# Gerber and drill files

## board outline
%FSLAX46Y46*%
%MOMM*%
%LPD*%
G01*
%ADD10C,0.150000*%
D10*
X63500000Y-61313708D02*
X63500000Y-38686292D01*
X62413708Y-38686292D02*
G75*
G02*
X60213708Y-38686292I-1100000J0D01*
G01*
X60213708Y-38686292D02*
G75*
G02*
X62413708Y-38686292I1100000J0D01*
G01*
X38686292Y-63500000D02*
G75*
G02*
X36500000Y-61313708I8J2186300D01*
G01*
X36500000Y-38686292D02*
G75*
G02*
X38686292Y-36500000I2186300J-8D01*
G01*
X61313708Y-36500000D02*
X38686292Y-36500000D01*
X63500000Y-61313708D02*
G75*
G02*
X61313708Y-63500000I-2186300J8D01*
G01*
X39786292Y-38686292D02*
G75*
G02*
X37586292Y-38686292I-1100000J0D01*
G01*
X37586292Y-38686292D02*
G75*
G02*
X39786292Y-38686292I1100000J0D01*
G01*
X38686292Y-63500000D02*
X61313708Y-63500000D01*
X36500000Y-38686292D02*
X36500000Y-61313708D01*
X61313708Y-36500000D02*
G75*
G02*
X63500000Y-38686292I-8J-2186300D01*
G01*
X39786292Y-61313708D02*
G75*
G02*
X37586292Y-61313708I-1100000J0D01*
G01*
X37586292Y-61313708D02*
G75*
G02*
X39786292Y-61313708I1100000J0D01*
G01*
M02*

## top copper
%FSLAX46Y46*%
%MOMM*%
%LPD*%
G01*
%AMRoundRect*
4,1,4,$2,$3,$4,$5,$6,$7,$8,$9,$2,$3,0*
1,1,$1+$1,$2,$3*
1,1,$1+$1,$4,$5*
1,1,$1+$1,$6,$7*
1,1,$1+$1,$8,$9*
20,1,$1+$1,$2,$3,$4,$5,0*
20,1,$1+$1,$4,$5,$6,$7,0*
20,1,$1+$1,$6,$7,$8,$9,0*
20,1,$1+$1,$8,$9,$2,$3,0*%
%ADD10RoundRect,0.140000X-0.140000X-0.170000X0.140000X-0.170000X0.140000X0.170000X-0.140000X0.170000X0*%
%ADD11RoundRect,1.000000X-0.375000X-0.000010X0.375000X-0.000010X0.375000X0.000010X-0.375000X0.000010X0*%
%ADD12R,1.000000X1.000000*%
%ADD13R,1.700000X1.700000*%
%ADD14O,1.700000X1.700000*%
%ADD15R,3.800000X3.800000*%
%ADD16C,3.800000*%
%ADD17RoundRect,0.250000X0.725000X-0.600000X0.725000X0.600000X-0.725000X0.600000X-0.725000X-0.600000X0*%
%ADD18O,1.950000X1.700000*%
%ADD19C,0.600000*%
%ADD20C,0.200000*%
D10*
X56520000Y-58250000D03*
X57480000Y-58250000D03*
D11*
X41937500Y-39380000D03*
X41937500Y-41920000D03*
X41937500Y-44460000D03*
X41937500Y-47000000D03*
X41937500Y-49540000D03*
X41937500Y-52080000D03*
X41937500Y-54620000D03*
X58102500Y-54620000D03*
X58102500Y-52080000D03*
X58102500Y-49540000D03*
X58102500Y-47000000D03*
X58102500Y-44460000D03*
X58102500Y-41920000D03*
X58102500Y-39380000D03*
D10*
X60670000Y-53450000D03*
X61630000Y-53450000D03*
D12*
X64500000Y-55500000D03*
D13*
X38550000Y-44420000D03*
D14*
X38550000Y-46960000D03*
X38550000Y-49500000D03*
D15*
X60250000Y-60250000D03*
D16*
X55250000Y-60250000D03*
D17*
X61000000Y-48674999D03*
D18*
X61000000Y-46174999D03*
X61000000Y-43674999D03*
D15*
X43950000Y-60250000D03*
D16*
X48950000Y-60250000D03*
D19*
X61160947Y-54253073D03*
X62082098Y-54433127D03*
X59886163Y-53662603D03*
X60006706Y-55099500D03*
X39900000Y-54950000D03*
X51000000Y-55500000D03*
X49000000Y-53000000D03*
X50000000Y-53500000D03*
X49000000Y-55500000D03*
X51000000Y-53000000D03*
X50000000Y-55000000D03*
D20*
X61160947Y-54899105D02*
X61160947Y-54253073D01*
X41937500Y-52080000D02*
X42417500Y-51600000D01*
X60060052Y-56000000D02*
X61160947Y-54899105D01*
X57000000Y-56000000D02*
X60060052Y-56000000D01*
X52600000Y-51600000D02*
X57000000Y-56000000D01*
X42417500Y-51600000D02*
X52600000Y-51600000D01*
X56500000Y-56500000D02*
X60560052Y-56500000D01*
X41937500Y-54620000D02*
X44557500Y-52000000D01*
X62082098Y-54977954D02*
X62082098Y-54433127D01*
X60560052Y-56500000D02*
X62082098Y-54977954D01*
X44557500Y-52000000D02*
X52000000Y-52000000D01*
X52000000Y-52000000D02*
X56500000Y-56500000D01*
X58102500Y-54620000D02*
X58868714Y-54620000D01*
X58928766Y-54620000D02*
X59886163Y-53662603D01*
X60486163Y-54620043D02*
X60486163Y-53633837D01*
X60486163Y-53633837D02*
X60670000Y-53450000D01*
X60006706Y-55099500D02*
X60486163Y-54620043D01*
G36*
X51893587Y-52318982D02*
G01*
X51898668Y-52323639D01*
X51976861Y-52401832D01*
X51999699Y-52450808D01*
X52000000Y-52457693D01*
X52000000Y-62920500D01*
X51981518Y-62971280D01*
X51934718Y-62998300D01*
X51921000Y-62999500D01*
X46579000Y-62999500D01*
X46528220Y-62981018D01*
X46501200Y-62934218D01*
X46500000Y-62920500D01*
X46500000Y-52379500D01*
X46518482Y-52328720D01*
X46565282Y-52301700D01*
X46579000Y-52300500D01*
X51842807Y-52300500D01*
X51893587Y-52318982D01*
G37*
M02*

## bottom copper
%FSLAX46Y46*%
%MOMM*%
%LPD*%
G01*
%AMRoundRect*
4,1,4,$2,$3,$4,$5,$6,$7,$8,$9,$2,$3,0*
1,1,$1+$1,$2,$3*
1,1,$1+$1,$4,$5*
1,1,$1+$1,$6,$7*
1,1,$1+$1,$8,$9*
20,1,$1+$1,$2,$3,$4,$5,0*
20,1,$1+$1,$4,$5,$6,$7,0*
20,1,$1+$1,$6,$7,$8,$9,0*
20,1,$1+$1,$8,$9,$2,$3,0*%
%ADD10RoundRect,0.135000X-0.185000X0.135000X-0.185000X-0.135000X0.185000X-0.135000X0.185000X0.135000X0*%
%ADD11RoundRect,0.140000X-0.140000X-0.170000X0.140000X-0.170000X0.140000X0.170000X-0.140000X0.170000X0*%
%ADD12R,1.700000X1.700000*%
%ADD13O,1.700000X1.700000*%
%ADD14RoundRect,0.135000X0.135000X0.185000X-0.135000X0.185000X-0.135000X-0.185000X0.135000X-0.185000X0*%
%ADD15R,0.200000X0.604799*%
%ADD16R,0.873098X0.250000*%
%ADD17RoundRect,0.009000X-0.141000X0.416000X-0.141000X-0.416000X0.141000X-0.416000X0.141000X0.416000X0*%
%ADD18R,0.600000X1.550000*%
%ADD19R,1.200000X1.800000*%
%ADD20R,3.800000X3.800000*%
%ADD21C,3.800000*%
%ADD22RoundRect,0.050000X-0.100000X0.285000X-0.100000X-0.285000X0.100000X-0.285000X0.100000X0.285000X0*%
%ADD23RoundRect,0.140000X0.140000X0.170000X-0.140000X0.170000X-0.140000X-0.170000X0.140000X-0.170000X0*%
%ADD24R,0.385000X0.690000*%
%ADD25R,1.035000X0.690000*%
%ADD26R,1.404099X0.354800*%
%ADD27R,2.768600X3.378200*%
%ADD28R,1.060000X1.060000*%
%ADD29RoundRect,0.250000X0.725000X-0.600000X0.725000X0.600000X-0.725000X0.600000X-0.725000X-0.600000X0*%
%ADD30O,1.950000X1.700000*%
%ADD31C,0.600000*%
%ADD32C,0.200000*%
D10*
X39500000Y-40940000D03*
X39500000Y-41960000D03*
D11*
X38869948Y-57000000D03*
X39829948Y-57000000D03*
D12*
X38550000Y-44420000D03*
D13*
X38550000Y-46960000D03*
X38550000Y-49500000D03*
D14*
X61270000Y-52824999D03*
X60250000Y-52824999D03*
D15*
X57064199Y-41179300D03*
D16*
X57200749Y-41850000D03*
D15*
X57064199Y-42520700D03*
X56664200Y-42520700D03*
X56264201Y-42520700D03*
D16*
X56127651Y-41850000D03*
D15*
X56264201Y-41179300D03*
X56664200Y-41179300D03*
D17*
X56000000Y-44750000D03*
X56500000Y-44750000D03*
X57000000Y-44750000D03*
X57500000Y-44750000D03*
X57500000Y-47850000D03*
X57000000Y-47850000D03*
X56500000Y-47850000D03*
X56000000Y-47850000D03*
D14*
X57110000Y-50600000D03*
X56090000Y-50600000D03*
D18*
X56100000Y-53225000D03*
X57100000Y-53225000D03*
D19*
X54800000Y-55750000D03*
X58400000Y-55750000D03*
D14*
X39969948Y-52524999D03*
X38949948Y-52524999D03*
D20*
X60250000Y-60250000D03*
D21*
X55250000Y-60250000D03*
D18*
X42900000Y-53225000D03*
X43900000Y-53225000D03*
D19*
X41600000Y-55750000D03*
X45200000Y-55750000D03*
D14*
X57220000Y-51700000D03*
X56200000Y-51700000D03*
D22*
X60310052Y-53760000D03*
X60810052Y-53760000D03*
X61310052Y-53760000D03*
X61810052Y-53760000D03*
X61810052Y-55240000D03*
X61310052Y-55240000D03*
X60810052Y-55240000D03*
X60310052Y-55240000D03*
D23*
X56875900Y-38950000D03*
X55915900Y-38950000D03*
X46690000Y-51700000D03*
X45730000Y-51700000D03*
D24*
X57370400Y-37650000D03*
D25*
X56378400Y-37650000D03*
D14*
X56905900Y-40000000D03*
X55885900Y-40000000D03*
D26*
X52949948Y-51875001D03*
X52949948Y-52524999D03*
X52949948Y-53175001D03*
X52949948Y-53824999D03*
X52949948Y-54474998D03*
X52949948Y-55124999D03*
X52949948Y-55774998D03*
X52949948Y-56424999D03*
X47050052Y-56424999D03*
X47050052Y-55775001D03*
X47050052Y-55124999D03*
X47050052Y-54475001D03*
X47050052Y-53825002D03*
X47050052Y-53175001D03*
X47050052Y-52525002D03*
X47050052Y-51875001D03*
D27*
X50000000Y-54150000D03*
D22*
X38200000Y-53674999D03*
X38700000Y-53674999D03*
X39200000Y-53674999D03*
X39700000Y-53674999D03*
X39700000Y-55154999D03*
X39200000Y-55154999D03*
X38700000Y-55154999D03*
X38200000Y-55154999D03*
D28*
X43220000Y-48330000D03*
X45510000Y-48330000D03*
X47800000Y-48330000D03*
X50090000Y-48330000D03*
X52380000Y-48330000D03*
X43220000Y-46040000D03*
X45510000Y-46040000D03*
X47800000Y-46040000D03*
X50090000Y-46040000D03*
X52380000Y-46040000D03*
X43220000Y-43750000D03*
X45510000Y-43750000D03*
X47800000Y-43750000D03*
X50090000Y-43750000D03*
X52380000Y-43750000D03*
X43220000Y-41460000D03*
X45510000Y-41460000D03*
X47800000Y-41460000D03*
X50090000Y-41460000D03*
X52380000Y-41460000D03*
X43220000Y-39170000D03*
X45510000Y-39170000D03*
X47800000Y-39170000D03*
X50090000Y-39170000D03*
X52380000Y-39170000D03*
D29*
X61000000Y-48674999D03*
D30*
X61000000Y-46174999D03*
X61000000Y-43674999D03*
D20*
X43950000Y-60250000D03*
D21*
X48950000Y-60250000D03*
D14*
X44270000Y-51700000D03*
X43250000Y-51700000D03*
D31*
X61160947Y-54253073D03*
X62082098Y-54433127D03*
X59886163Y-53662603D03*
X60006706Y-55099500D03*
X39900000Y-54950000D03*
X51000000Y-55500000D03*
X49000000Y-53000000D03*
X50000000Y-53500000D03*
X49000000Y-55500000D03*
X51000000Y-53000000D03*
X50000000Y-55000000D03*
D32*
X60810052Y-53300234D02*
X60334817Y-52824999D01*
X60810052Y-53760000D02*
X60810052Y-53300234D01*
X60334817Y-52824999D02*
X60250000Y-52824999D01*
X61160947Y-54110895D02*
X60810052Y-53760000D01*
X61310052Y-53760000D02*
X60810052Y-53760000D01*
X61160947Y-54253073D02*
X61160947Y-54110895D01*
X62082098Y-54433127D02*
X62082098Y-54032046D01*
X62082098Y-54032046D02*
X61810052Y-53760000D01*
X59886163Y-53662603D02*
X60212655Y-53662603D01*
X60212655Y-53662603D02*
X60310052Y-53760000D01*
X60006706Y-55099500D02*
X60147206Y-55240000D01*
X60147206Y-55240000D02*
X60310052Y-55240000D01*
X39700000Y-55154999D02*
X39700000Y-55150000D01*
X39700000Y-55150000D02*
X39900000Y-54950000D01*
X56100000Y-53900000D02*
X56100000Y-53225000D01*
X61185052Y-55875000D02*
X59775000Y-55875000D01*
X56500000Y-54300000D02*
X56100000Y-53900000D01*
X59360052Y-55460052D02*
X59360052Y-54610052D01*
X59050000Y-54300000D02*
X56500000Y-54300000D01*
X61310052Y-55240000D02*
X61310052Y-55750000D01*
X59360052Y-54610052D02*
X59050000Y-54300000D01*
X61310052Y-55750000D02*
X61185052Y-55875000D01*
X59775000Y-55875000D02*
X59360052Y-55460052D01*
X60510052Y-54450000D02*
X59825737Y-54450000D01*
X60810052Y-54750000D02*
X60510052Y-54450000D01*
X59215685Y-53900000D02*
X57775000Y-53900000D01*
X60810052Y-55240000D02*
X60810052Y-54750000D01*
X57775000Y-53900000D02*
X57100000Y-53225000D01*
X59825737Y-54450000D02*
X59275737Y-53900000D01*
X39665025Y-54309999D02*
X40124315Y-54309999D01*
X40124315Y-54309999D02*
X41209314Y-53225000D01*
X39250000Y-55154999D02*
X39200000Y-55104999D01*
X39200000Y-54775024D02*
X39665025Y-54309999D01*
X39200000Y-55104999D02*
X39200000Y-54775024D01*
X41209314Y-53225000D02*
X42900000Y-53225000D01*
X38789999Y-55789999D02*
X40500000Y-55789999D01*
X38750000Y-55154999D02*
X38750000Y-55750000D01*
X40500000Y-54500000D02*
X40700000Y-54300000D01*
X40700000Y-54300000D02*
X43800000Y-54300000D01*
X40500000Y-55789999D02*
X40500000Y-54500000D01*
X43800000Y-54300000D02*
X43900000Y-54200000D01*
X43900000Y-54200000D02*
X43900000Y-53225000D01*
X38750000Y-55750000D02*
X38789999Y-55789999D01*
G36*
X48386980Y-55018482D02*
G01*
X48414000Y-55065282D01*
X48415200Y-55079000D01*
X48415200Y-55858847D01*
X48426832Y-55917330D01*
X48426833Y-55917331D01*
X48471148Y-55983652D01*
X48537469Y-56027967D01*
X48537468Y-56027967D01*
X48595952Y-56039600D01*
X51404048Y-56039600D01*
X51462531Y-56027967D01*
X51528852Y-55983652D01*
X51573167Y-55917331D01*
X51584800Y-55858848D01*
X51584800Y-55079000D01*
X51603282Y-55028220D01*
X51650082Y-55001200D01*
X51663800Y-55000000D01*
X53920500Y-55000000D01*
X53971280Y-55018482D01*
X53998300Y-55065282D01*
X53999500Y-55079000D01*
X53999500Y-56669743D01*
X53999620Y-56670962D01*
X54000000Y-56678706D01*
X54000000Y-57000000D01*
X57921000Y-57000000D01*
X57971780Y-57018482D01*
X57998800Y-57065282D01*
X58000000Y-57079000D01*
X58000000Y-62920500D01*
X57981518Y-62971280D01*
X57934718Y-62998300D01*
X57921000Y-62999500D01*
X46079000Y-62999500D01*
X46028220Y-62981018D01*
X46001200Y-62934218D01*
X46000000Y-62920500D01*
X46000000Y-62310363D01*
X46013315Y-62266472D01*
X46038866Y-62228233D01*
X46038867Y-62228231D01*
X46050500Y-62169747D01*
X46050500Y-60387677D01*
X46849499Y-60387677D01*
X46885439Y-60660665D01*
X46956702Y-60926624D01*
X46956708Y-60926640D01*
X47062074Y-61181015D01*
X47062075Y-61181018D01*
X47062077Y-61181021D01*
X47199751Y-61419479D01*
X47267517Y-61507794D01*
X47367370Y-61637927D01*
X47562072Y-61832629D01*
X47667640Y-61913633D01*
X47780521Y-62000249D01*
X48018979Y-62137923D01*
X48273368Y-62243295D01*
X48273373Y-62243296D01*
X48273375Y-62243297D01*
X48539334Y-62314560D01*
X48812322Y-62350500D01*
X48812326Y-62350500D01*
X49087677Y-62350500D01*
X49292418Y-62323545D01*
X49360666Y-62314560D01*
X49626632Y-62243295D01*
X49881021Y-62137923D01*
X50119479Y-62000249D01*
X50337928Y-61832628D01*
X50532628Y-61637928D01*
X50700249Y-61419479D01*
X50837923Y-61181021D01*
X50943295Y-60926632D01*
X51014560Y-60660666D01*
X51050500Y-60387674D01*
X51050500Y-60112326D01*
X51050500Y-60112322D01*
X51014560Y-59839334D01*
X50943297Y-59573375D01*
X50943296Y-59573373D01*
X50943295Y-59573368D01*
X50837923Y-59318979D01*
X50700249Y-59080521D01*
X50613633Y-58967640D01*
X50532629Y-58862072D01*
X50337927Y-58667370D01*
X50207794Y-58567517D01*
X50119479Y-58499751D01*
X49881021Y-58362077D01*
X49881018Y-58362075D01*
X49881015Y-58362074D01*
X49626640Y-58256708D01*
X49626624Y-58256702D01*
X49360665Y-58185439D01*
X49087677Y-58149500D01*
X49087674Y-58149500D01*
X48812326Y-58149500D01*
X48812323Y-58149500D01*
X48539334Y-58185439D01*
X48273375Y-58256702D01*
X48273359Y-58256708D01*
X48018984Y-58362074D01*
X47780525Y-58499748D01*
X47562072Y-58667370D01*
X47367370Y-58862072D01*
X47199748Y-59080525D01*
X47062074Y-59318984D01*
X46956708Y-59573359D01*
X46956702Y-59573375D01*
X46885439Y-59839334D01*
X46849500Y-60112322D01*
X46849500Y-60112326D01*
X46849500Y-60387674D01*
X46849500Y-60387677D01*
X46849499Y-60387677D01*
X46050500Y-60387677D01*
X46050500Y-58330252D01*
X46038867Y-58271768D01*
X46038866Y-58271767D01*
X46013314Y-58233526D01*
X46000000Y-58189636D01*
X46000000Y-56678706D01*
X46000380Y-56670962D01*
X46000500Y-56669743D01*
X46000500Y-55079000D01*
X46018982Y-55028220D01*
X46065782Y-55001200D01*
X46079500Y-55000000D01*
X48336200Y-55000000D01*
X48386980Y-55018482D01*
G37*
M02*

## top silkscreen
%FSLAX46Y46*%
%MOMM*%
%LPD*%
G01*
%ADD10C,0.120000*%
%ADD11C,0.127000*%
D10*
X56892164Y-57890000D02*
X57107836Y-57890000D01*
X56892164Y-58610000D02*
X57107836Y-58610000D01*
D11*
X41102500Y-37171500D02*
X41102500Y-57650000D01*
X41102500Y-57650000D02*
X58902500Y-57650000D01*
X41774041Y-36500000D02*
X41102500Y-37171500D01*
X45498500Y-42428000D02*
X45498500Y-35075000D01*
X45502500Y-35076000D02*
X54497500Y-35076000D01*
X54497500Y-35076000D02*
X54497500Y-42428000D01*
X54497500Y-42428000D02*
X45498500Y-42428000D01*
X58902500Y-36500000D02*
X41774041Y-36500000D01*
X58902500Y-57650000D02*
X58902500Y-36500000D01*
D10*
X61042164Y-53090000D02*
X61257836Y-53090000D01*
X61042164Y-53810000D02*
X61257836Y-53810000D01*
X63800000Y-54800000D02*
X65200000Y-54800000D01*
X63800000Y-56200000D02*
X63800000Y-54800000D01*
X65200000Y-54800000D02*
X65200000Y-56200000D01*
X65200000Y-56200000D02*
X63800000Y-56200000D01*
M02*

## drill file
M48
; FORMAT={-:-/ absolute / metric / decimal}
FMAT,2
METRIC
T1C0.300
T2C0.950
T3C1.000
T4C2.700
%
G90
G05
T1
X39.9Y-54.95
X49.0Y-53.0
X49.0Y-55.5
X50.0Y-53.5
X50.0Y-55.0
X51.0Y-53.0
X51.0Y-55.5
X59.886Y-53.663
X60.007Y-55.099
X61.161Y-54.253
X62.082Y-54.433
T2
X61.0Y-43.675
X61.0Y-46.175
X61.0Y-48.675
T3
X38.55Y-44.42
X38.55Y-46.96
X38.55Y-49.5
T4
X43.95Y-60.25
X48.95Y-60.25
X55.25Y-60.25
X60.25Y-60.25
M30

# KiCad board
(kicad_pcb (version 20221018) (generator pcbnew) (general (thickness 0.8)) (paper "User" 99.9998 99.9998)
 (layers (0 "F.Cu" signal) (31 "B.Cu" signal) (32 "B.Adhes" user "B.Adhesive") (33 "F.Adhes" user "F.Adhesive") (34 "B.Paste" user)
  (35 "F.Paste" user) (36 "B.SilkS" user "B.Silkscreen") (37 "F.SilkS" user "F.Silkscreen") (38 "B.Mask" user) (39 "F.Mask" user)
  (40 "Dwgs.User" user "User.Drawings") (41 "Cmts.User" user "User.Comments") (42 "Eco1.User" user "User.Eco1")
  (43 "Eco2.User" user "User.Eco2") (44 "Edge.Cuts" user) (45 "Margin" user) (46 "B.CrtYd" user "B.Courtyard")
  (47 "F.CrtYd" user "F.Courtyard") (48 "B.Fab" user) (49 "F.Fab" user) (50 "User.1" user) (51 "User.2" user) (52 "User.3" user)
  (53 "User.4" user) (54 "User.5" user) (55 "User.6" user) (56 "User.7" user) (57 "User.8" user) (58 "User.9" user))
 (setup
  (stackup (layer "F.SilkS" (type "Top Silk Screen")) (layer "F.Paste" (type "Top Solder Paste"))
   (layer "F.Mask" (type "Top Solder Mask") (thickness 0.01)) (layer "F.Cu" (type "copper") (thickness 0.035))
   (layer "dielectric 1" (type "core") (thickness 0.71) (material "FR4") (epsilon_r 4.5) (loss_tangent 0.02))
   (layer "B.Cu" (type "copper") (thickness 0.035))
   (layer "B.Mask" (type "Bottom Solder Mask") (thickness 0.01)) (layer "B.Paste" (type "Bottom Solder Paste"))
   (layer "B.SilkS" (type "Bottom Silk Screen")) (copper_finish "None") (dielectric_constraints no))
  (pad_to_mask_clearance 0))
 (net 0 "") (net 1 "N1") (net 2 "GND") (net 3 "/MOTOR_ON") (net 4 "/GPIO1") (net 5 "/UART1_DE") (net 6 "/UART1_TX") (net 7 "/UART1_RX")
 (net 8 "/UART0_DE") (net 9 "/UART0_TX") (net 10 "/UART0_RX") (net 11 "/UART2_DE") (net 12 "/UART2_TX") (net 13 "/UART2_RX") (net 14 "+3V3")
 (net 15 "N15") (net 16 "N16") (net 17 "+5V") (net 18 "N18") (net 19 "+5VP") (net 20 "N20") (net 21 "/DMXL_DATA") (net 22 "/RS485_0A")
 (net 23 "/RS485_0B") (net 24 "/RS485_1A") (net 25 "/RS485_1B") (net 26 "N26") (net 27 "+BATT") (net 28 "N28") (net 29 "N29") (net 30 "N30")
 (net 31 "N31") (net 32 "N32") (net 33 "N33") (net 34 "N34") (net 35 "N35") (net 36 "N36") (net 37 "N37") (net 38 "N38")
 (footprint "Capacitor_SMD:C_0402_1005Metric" (layer "F.Cu") (at 57 58.25)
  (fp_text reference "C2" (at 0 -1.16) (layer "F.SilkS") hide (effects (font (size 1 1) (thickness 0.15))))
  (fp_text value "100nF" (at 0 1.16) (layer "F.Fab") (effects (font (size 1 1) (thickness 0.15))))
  (fp_line (start -0.107836 -0.36) (end 0.107836 -0.36) (stroke (width 0.12) (type solid)) (layer "F.SilkS"))
  (fp_line (start -0.107836 0.36) (end 0.107836 0.36) (stroke (width 0.12) (type solid)) (layer "F.SilkS"))
  (pad "1" smd roundrect (at -0.48 0) (size 0.56 0.62) (layers "F.Cu" "F.Paste" "F.Mask") (roundrect_rratio 0.25) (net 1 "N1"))
  (pad "2" smd roundrect (at 0.48 0) (size 0.56 0.62) (layers "F.Cu" "F.Paste" "F.Mask") (roundrect_rratio 0.25) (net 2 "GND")))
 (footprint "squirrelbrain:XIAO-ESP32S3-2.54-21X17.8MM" (layer "F.Cu") (at 50 36.5)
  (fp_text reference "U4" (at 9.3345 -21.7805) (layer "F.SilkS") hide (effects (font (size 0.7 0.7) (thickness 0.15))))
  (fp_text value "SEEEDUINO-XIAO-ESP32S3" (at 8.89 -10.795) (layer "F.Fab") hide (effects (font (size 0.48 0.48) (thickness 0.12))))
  (fp_line (start -8.8975 0.6715) (end -8.8975 21.15) (stroke (width 0.127) (type solid)) (layer "F.SilkS"))
  (fp_line (start -8.8975 21.15) (end 8.9025 21.15) (stroke (width 0.127) (type solid)) (layer "F.SilkS"))
  (fp_line (start -8.225959 0) (end -8.8975 0.6715) (stroke (width 0.127) (type solid)) (layer "F.SilkS"))
  (fp_line (start -4.5015 5.928) (end -4.5015 -1.425) (stroke (width 0.127) (type solid)) (layer "F.SilkS"))
  (fp_line (start -4.4975 -1.424) (end 4.4975 -1.424) (stroke (width 0.127) (type solid)) (layer "F.SilkS"))
  (fp_line (start 4.4975 -1.424) (end 4.4975 5.928) (stroke (width 0.127) (type solid)) (layer "F.SilkS"))
  (fp_line (start 4.4975 5.928) (end -4.5015 5.928) (stroke (width 0.127) (type solid)) (layer "F.SilkS"))
  (fp_line (start 8.9025 0) (end -8.225959 0) (stroke (width 0.127) (type solid)) (layer "F.SilkS"))
  (fp_line (start 8.9025 21.15) (end 8.9025 0) (stroke (width 0.127) (type solid)) (layer "F.SilkS"))
  (pad "1" smd roundrect (at -8.0625 2.88) (size 2.75 2) (layers "F.Cu" "F.Paste" "F.Mask") (roundrect_rratio 0.5) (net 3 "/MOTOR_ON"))
  (pad "2" smd roundrect (at -8.0625 5.42) (size 2.75 2) (layers "F.Cu" "F.Paste" "F.Mask") (roundrect_rratio 0.5) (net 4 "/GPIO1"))
  (pad "3" smd roundrect (at -8.0625 7.96) (size 2.75 2) (layers "F.Cu" "F.Paste" "F.Mask") (roundrect_rratio 0.5) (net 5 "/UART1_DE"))
  (pad "4" smd roundrect (at -8.0625 10.5) (size 2.75 2) (layers "F.Cu" "F.Paste" "F.Mask") (roundrect_rratio 0.5) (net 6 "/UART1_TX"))
  (pad "5" smd roundrect (at -8.0625 13.04) (size 2.75 2) (layers "F.Cu" "F.Paste" "F.Mask") (roundrect_rratio 0.5) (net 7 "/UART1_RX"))
  (pad "6" smd roundrect (at -8.0625 15.58) (size 2.75 2) (layers "F.Cu" "F.Paste" "F.Mask") (roundrect_rratio 0.5) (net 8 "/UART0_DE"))
  (pad "7" smd roundrect (at -8.0625 18.12) (size 2.75 2) (layers "F.Cu" "F.Paste" "F.Mask") (roundrect_rratio 0.5) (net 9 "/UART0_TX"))
  (pad "8" smd roundrect (at 8.1025 18.12) (size 2.75 2) (layers "F.Cu" "F.Paste" "F.Mask") (roundrect_rratio 0.5) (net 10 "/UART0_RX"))
  (pad "9" smd roundrect (at 8.1025 15.58) (size 2.75 2) (layers "F.Cu" "F.Paste" "F.Mask") (roundrect_rratio 0.5) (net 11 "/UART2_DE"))
  (pad "10" smd roundrect (at 8.1025 13.04) (size 2.75 2) (layers "F.Cu" "F.Paste" "F.Mask") (roundrect_rratio 0.5) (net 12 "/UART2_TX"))
  (pad "11" smd roundrect (at 8.1025 10.5) (size 2.75 2) (layers "F.Cu" "F.Paste" "F.Mask") (roundrect_rratio 0.5) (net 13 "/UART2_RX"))
  (pad "12" smd roundrect (at 8.1025 7.96) (size 2.75 2) (layers "F.Cu" "F.Paste" "F.Mask") (roundrect_rratio 0.5) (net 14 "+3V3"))
  (pad "13" smd roundrect (at 8.1025 5.42) (size 2.75 2) (layers "F.Cu" "F.Paste" "F.Mask") (roundrect_rratio 0.5) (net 2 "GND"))
  (pad "14" smd roundrect (at 8.1025 2.88) (size 2.75 2) (layers "F.Cu" "F.Paste" "F.Mask") (roundrect_rratio 0.5) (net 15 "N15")))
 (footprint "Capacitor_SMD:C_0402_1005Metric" (layer "F.Cu") (at 61.15 53.45)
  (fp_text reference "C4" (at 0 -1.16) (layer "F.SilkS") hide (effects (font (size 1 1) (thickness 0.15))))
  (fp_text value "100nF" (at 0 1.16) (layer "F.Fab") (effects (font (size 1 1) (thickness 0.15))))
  (fp_line (start -0.107836 -0.36) (end 0.107836 -0.36) (stroke (width 0.12) (type solid)) (layer "F.SilkS"))
  (fp_line (start -0.107836 0.36) (end 0.107836 0.36) (stroke (width 0.12) (type solid)) (layer "F.SilkS"))
  (pad "1" smd roundrect (at -0.48 0) (size 0.56 0.62) (layers "F.Cu" "F.Paste" "F.Mask") (roundrect_rratio 0.25) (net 14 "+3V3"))
  (pad "2" smd roundrect (at 0.48 0) (size 0.56 0.62) (layers "F.Cu" "F.Paste" "F.Mask") (roundrect_rratio 0.25) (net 2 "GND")))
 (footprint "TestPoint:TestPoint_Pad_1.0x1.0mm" (layer "F.Cu") (at 64.5 55.5)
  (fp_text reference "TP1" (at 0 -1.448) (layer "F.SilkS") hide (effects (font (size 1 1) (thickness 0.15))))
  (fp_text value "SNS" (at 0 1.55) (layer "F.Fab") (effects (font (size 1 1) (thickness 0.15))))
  (fp_line (start -0.7 -0.7) (end 0.7 -0.7) (stroke (width 0.12) (type solid)) (layer "F.SilkS"))
  (fp_line (start -0.7 0.7) (end -0.7 -0.7) (stroke (width 0.12) (type solid)) (layer "F.SilkS"))
  (fp_line (start 0.7 -0.7) (end 0.7 0.7) (stroke (width 0.12) (type solid)) (layer "F.SilkS"))
  (fp_line (start 0.7 0.7) (end -0.7 0.7) (stroke (width 0.12) (type solid)) (layer "F.SilkS"))
  (pad "1" smd rect (at 0 0) (size 1 1) (layers "F.Cu" "F.Mask") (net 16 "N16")))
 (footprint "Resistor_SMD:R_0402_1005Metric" (layer "B.Cu") (at 39.5 41.45 -90)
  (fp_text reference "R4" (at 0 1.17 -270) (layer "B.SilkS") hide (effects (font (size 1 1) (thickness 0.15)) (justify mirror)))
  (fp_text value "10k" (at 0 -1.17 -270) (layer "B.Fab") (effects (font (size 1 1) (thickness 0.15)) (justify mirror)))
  (pad "1" smd roundrect (at -0.51 0 270) (size 0.54 0.64) (layers "B.Cu" "B.Paste" "B.Mask") (roundrect_rratio 0.25) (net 2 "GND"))
  (pad "2" smd roundrect (at 0.51 0 270) (size 0.54 0.64) (layers "B.Cu" "B.Paste" "B.Mask") (roundrect_rratio 0.25) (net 3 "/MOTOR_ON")))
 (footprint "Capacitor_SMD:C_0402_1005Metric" (layer "B.Cu") (at 39.349948 57)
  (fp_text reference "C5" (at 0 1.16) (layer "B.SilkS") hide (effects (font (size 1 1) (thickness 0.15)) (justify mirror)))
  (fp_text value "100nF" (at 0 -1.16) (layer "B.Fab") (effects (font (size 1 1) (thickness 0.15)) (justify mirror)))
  (pad "1" smd roundrect (at -0.48 0) (size 0.56 0.62) (layers "B.Cu" "B.Paste" "B.Mask") (roundrect_rratio 0.25) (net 14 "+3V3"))
  (pad "2" smd roundrect (at 0.48 0) (size 0.56 0.62) (layers "B.Cu" "B.Paste" "B.Mask") (roundrect_rratio 0.25) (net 2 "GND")))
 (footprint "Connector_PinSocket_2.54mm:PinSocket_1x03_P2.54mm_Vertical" (layer "B.Cu") (at 38.55 44.42 180)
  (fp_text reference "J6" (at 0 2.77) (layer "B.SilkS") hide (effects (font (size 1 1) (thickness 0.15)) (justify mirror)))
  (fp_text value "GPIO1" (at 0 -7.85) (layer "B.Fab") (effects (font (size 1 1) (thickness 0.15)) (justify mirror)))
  (pad "1" thru_hole rect (at 0 0 180) (size 1.7 1.7) (drill 1) (layers "*.Cu" "*.Mask") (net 4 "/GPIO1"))
  (pad "2" thru_hole oval (at 0 -2.54 180) (size 1.7 1.7) (drill 1) (layers "*.Cu" "*.Mask") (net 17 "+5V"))
  (pad "3" thru_hole oval (at 0 -5.08 180) (size 1.7 1.7) (drill 1) (layers "*.Cu" "*.Mask") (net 2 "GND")))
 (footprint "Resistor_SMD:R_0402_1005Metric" (layer "B.Cu") (at 60.76 52.824999 180)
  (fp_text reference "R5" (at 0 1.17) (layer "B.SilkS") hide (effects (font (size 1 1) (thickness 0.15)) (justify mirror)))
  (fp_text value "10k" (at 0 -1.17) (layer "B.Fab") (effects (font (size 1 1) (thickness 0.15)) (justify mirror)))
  (pad "1" smd roundrect (at -0.51 0 180) (size 0.54 0.64) (layers "B.Cu" "B.Paste" "B.Mask") (roundrect_rratio 0.25) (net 2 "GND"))
  (pad "2" smd roundrect (at 0.51 0 180) (size 0.54 0.64) (layers "B.Cu" "B.Paste" "B.Mask") (roundrect_rratio 0.25) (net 8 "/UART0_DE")))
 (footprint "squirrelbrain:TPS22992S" (layer "B.Cu") (at 56.6642 41.85 180)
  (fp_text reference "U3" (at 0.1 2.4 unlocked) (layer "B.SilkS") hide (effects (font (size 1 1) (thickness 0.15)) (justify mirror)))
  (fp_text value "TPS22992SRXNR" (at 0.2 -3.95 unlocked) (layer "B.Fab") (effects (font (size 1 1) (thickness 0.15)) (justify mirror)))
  (pad "1" smd rect (at -0.399999 0.6707 180) (size 0.2 0.604799) (layers "B.Cu" "B.Paste" "B.Mask") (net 17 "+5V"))
  (pad "2" smd rect (at -0.536549 0 90) (size 0.25 0.873098) (layers "B.Cu" "B.Paste" "B.Mask") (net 17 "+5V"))
  (pad "3" smd rect (at -0.399999 -0.6707 180) (size 0.2 0.604799) (layers "B.Cu" "B.Paste" "B.Mask") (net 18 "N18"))
  (pad "4" smd rect (at 0 -0.6707 180) (size 0.2 0.604799) (layers "B.Cu" "B.Paste" "B.Mask") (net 2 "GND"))
  (pad "5" smd rect (at 0.399999 -0.6707 180) (size 0.2 0.604799) (layers "B.Cu" "B.Paste" "B.Mask") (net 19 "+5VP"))
  (pad "6" smd rect (at 0.536549 0 90) (size 0.25 0.873098) (layers "B.Cu" "B.Paste" "B.Mask") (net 19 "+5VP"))
  (pad "7" smd rect (at 0.399999 0.6707 180) (size 0.2 0.604799) (layers "B.Cu" "B.Paste" "B.Mask") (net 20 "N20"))
  (pad "8" smd rect (at 0 0.6707 180) (size 0.2 0.604799) (layers "B.Cu" "B.Paste" "B.Mask") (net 3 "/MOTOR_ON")))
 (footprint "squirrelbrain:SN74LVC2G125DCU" (layer "B.Cu") (at 56.75 46.3 -90)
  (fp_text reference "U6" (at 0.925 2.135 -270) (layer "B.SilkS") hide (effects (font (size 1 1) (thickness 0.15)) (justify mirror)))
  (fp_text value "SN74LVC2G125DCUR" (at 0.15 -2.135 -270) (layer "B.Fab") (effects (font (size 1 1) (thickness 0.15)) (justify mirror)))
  (pad "1" smd roundrect (at -1.55 0.75 270) (size 0.85 0.3) (layers "B.Cu" "B.Paste" "B.Mask") (roundrect_rratio 0.03) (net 11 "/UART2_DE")
   (solder_mask_margin 0.05))
  (pad "2" smd roundrect (at -1.55 0.25 270) (size 0.85 0.3) (layers "B.Cu" "B.Paste" "B.Mask") (roundrect_rratio 0.03)
   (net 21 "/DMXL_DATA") (solder_mask_margin 0.05))
  (pad "3" smd roundrect (at -1.55 -0.25 270) (size 0.85 0.3) (layers "B.Cu" "B.Paste" "B.Mask") (roundrect_rratio 0.03)
   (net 21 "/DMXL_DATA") (solder_mask_margin 0.05))
  (pad "4" smd roundrect (at -1.55 -0.75 270) (size 0.85 0.3) (layers "B.Cu" "B.Paste" "B.Mask") (roundrect_rratio 0.03) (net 2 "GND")
   (solder_mask_margin 0.05))
  (pad "5" smd roundrect (at 1.55 -0.75 270) (size 0.85 0.3) (layers "B.Cu" "B.Paste" "B.Mask") (roundrect_rratio 0.03) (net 12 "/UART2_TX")
   (solder_mask_margin 0.05))
  (pad "6" smd roundrect (at 1.55 -0.25 270) (size 0.85 0.3) (layers "B.Cu" "B.Paste" "B.Mask") (roundrect_rratio 0.03) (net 13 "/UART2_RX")
   (solder_mask_margin 0.05))
  (pad "7" smd roundrect (at 1.55 0.25 270) (size 0.85 0.3) (layers "B.Cu" "B.Paste" "B.Mask") (roundrect_rratio 0.03) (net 11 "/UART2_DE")
   (solder_mask_margin 0.05))
  (pad "8" smd roundrect (at 1.55 0.75 270) (size 0.85 0.3) (layers "B.Cu" "B.Paste" "B.Mask") (roundrect_rratio 0.03) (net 14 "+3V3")
   (solder_mask_margin 0.05)))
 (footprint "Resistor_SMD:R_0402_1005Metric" (layer "B.Cu") (at 56.6 50.6 180)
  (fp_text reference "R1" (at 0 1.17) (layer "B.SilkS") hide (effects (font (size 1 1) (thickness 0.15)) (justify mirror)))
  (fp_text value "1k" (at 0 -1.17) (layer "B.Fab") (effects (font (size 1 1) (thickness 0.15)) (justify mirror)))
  (pad "1" smd roundrect (at -0.51 0 180) (size 0.54 0.64) (layers "B.Cu" "B.Paste" "B.Mask") (roundrect_rratio 0.25) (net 2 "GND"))
  (pad "2" smd roundrect (at 0.51 0 180) (size 0.54 0.64) (layers "B.Cu" "B.Paste" "B.Mask") (roundrect_rratio 0.25) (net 16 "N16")))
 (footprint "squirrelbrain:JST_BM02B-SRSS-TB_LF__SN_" (layer "B.Cu") (at 56.6 55.75)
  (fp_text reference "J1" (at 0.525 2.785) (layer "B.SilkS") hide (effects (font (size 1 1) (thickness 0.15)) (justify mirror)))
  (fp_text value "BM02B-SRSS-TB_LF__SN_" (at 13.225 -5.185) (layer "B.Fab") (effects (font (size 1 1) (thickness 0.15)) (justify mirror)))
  (pad "1" smd rect (at -0.5 -2.525) (size 0.6 1.55) (layers "B.Cu" "B.Paste" "B.Mask") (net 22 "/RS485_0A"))
  (pad "2" smd rect (at 0.5 -2.525) (size 0.6 1.55) (layers "B.Cu" "B.Paste" "B.Mask") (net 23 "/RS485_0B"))
  (pad "S1" smd rect (at -1.8 0) (size 1.2 1.8) (layers "B.Cu" "B.Paste" "B.Mask") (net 2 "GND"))
  (pad "S2" smd rect (at 1.8 0) (size 1.2 1.8) (layers "B.Cu" "B.Paste" "B.Mask") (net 2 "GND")))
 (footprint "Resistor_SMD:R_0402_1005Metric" (layer "B.Cu") (at 39.459948 52.524999 180)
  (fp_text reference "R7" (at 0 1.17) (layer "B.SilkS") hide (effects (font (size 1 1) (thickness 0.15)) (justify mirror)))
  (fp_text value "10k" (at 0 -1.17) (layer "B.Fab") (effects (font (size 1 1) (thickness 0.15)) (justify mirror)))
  (pad "1" smd roundrect (at -0.51 0 180) (size 0.54 0.64) (layers "B.Cu" "B.Paste" "B.Mask") (roundrect_rratio 0.25) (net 2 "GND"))
  (pad "2" smd roundrect (at 0.51 0 180) (size 0.54 0.64) (layers "B.Cu" "B.Paste" "B.Mask") (roundrect_rratio 0.25) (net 5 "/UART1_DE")))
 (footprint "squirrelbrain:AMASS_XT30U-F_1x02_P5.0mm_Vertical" (layer "B.Cu") (at 60.25 60.25 180)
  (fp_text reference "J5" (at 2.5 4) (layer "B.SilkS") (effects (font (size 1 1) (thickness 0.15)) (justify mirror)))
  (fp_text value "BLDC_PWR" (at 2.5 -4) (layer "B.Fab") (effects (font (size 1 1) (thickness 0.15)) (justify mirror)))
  (pad "1" thru_hole rect (at 0 0 180) (size 3.8 3.8) (drill 2.7) (layers "*.Cu" "*.Mask") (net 2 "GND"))
  (pad "2" thru_hole circle (at 5 0 180) (size 3.8 3.8) (drill 2.7) (layers "*.Cu" "*.Mask") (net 1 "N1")))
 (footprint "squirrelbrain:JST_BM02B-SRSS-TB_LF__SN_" (layer "B.Cu") (at 43.4 55.75)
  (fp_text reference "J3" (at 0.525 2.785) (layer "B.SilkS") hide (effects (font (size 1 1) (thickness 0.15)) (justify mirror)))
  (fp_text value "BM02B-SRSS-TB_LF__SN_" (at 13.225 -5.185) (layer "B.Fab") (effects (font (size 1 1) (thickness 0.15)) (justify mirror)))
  (pad "1" smd rect (at -0.5 -2.525) (size 0.6 1.55) (layers "B.Cu" "B.Paste" "B.Mask") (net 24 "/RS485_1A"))
  (pad "2" smd rect (at 0.5 -2.525) (size 0.6 1.55) (layers "B.Cu" "B.Paste" "B.Mask") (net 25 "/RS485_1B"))
  (pad "S1" smd rect (at -1.8 0) (size 1.2 1.8) (layers "B.Cu" "B.Paste" "B.Mask") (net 2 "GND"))
  (pad "S2" smd rect (at 1.8 0) (size 1.2 1.8) (layers "B.Cu" "B.Paste" "B.Mask") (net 2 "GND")))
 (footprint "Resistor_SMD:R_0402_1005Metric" (layer "B.Cu") (at 56.71 51.7 180)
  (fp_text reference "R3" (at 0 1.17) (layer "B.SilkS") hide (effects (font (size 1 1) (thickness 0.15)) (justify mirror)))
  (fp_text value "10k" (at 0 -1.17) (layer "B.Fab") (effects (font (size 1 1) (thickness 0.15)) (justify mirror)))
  (pad "1" smd roundrect (at -0.51 0 180) (size 0.54 0.64) (layers "B.Cu" "B.Paste" "B.Mask") (roundrect_rratio 0.25) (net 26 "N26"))
  (pad "2" smd roundrect (at 0.51 0 180) (size 0.54 0.64) (layers "B.Cu" "B.Paste" "B.Mask") (roundrect_rratio 0.25) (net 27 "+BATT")))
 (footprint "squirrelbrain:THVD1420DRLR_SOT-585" (layer "B.Cu") (at 61.060052 54.5 -90)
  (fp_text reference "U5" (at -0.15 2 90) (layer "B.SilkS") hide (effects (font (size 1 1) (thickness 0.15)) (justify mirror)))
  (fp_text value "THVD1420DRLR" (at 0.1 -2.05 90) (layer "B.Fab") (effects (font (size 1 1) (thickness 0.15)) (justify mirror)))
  (pad "1" smd roundrect (at -0.74 0.75 270) (size 0.67 0.3) (layers "B.Cu" "B.Paste" "B.Mask") (roundrect_rratio 0.1666666667)
   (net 10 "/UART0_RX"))
  (pad "2" smd roundrect (at -0.74 0.25 270) (size 0.67 0.3) (layers "B.Cu" "B.Paste" "B.Mask") (roundrect_rratio 0.1666666667)
   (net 8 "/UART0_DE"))
  (pad "3" smd roundrect (at -0.74 -0.25 270) (size 0.67 0.3) (layers "B.Cu" "B.Paste" "B.Mask") (roundrect_rratio 0.1666666667)
   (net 8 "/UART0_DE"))
  (pad "4" smd roundrect (at -0.74 -0.75 270) (size 0.67 0.3) (layers "B.Cu" "B.Paste" "B.Mask") (roundrect_rratio 0.1666666667)
   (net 9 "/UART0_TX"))
  (pad "5" smd roundrect (at 0.74 -0.75 270) (size 0.67 0.3) (layers "B.Cu" "B.Paste" "B.Mask") (roundrect_rratio 0.1666666667)
   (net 2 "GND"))
  (pad "6" smd roundrect (at 0.74 -0.25 270) (size 0.67 0.3) (layers "B.Cu" "B.Paste" "B.Mask") (roundrect_rratio 0.1666666667)
   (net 22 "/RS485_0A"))
  (pad "7" smd roundrect (at 0.74 0.25 270) (size 0.67 0.3) (layers "B.Cu" "B.Paste" "B.Mask") (roundrect_rratio 0.1666666667)
   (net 23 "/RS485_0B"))
  (pad "8" smd roundrect (at 0.74 0.75 270) (size 0.67 0.3) (layers "B.Cu" "B.Paste" "B.Mask") (roundrect_rratio 0.1666666667)
   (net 14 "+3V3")))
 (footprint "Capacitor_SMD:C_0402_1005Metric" (layer "B.Cu") (at 56.3959 38.95 180)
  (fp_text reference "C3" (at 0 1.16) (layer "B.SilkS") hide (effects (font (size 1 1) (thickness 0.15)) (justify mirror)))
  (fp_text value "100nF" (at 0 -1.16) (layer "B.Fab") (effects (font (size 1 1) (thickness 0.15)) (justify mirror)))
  (pad "1" smd roundrect (at -0.48 0 180) (size 0.56 0.62) (layers "B.Cu" "B.Paste" "B.Mask") (roundrect_rratio 0.25) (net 14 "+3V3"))
  (pad "2" smd roundrect (at 0.48 0 180) (size 0.56 0.62) (layers "B.Cu" "B.Paste" "B.Mask") (roundrect_rratio 0.25) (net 2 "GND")))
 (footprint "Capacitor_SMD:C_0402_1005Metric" (layer "B.Cu") (at 46.21 51.7 180)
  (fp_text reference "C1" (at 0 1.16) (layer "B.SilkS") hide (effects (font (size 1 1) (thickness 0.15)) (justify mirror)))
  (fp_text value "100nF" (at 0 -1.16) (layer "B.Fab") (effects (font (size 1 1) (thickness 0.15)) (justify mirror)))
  (pad "1" smd roundrect (at -0.48 0 180) (size 0.56 0.62) (layers "B.Cu" "B.Paste" "B.Mask") (roundrect_rratio 0.25) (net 27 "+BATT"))
  (pad "2" smd roundrect (at 0.48 0 180) (size 0.56 0.62) (layers "B.Cu" "B.Paste" "B.Mask") (roundrect_rratio 0.25) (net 2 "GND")))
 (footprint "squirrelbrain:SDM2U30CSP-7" (layer "B.Cu") (at 56.6959 37.65 180)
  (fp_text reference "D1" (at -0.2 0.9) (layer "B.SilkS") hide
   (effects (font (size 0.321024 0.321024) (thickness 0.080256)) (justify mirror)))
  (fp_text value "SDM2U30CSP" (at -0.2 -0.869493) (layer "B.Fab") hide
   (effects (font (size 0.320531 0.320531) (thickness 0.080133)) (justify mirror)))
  (pad "1" smd rect (at -0.6745 0 180) (size 0.385 0.69) (layers "B.Cu" "B.Paste" "B.Mask") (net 15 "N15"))
  (pad "2" smd rect (at 0.3175 0 180) (size 1.035 0.69) (layers "B.Cu" "B.Paste" "B.Mask") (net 17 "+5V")))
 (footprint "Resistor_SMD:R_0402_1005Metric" (layer "B.Cu") (at 56.3959 40 180)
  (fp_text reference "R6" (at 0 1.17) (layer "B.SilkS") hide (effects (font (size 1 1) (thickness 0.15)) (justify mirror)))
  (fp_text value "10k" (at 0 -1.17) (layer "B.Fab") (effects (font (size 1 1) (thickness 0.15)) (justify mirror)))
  (pad "1" smd roundrect (at -0.51 0 180) (size 0.54 0.64) (layers "B.Cu" "B.Paste" "B.Mask") (roundrect_rratio 0.25) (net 2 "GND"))
  (pad "2" smd roundrect (at 0.51 0 180) (size 0.54 0.64) (layers "B.Cu" "B.Paste" "B.Mask") (roundrect_rratio 0.25) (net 11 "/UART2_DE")))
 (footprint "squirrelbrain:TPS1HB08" (layer "B.Cu") (at 50 54.15 180)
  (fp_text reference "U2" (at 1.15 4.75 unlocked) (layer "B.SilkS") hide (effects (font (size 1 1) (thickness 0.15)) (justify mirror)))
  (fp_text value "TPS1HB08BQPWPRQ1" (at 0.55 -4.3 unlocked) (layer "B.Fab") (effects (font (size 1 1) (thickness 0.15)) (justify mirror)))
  (pad "1" smd rect (at -2.949948 2.274999 180) (size 1.404099 0.3548) (layers "B.Cu" "B.Paste" "B.Mask") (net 2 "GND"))
  (pad "2" smd rect (at -2.949948 1.625001 180) (size 1.404099 0.3548) (layers "B.Cu" "B.Paste" "B.Mask") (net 16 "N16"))
  (pad "3" smd rect (at -2.949948 0.974999 180) (size 1.404099 0.3548) (layers "B.Cu" "B.Paste" "B.Mask") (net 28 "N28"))
  (pad "4" smd rect (at -2.949948 0.325001 180) (size 1.404099 0.3548) (layers "B.Cu" "B.Paste" "B.Mask") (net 3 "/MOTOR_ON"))
  (pad "5" smd rect (at -2.949948 -0.324998 180) (size 1.404099 0.3548) (layers "B.Cu" "B.Paste" "B.Mask") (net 26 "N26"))
  (pad "6" smd rect (at -2.949948 -0.974999 180) (size 1.404099 0.3548) (layers "B.Cu" "B.Paste" "B.Mask") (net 1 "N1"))
  (pad "7" smd rect (at -2.949948 -1.624998 180) (size 1.404099 0.3548) (layers "B.Cu" "B.Paste" "B.Mask") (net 1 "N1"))
  (pad "8" smd rect (at -2.949948 -2.274999 180) (size 1.404099 0.3548) (layers "B.Cu" "B.Paste" "B.Mask") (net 1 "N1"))
  (pad "9" smd rect (at 2.949948 -2.274999 180) (size 1.404099 0.3548) (layers "B.Cu" "B.Paste" "B.Mask") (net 1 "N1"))
  (pad "10" smd rect (at 2.949948 -1.625001 180) (size 1.404099 0.3548) (layers "B.Cu" "B.Paste" "B.Mask") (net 1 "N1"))
  (pad "11" smd rect (at 2.949948 -0.974999 180) (size 1.404099 0.3548) (layers "B.Cu" "B.Paste" "B.Mask") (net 1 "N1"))
  (pad "12" smd rect (at 2.949948 -0.325001 180) (size 1.404099 0.3548) (layers "B.Cu" "B.Paste" "B.Mask") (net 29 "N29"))
  (pad "13" smd rect (at 2.949948 0.324998 180) (size 1.404099 0.3548) (layers "B.Cu" "B.Paste" "B.Mask") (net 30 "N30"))
  (pad "14" smd rect (at 2.949948 0.974999 180) (size 1.404099 0.3548) (layers "B.Cu" "B.Paste" "B.Mask") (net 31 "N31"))
  (pad "15" smd rect (at 2.949948 1.624998 180) (size 1.404099 0.3548) (layers "B.Cu" "B.Paste" "B.Mask") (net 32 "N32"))
  (pad "16" smd rect (at 2.949948 2.274999 180) (size 1.404099 0.3548) (layers "B.Cu" "B.Paste" "B.Mask") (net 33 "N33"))
  (pad "EPAD" smd rect (at 0 0 180) (size 2.7686 3.3782) (layers "B.Cu" "B.Mask") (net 27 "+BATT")))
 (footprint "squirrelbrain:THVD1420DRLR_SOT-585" (layer "B.Cu") (at 38.95 54.414999 -90)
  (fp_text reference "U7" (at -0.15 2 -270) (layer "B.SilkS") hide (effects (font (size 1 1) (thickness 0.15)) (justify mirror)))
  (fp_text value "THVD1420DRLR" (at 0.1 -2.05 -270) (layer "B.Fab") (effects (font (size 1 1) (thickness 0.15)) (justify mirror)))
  (pad "1" smd roundrect (at -0.74 0.75 270) (size 0.67 0.3) (layers "B.Cu" "B.Paste" "B.Mask") (roundrect_rratio 0.1666666667)
   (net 7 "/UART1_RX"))
  (pad "2" smd roundrect (at -0.74 0.25 270) (size 0.67 0.3) (layers "B.Cu" "B.Paste" "B.Mask") (roundrect_rratio 0.1666666667)
   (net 5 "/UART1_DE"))
  (pad "3" smd roundrect (at -0.74 -0.25 270) (size 0.67 0.3) (layers "B.Cu" "B.Paste" "B.Mask") (roundrect_rratio 0.1666666667)
   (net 5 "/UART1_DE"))
  (pad "4" smd roundrect (at -0.74 -0.75 270) (size 0.67 0.3) (layers "B.Cu" "B.Paste" "B.Mask") (roundrect_rratio 0.1666666667)
   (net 6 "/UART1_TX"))
  (pad "5" smd roundrect (at 0.74 -0.75 270) (size 0.67 0.3) (layers "B.Cu" "B.Paste" "B.Mask") (roundrect_rratio 0.1666666667)
   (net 2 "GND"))
  (pad "6" smd roundrect (at 0.74 -0.25 270) (size 0.67 0.3) (layers "B.Cu" "B.Paste" "B.Mask") (roundrect_rratio 0.1666666667)
   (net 24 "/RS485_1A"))
  (pad "7" smd roundrect (at 0.74 0.25 270) (size 0.67 0.3) (layers "B.Cu" "B.Paste" "B.Mask") (roundrect_rratio 0.1666666667)
   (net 25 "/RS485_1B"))
  (pad "8" smd roundrect (at 0.74 0.75 270) (size 0.67 0.3) (layers "B.Cu" "B.Paste" "B.Mask") (roundrect_rratio 0.1666666667)
   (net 14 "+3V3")))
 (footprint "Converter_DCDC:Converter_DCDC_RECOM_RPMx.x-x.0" (layer "B.Cu") (at 47.8 43.75)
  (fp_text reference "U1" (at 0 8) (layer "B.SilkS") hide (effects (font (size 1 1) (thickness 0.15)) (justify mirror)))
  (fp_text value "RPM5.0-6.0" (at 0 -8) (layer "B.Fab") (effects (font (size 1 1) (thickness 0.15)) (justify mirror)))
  (pad "A1" smd rect (at -4.58 4.58) (size 1.06 1.06) (layers "B.Cu" "B.Paste" "B.Mask") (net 27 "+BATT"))
  (pad "A2" smd rect (at -2.29 4.58) (size 1.06 1.06) (layers "B.Cu" "B.Paste" "B.Mask") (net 27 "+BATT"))
  (pad "A3" smd rect (at 0 4.58) (size 1.06 1.06) (layers "B.Cu" "B.Paste" "B.Mask") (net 2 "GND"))
  (pad "A4" smd rect (at 2.29 4.58) (size 1.06 1.06) (layers "B.Cu" "B.Paste" "B.Mask") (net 2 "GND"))
  (pad "A5" smd rect (at 4.58 4.58) (size 1.06 1.06) (layers "B.Cu" "B.Paste" "B.Mask") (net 17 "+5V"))
  (pad "B1" smd rect (at -4.58 2.29) (size 1.06 1.06) (layers "B.Cu" "B.Paste" "B.Mask") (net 2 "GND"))
  (pad "B2" smd rect (at -2.29 2.29) (size 1.06 1.06) (layers "B.Cu" "B.Paste" "B.Mask") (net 2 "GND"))
  (pad "B3" smd rect (at 0 2.29) (size 1.06 1.06) (layers "B.Cu" "B.Paste" "B.Mask") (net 2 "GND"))
  (pad "B4" smd rect (at 2.29 2.29) (size 1.06 1.06) (layers "B.Cu" "B.Paste" "B.Mask") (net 2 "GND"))
  (pad "B5" smd rect (at 4.58 2.29) (size 1.06 1.06) (layers "B.Cu" "B.Paste" "B.Mask") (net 17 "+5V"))
  (pad "C1" smd rect (at -4.58 0) (size 1.06 1.06) (layers "B.Cu" "B.Paste" "B.Mask") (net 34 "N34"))
  (pad "C2" smd rect (at -2.29 0) (size 1.06 1.06) (layers "B.Cu" "B.Paste" "B.Mask") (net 2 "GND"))
  (pad "C3" smd rect (at 0 0) (size 1.06 1.06) (layers "B.Cu" "B.Paste" "B.Mask") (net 2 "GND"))
  (pad "C4" smd rect (at 2.29 0) (size 1.06 1.06) (layers "B.Cu" "B.Paste" "B.Mask") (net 2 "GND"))
  (pad "C5" smd rect (at 4.58 0) (size 1.06 1.06) (layers "B.Cu" "B.Paste" "B.Mask") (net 17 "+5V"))
  (pad "D1" smd rect (at -4.58 -2.29) (size 1.06 1.06) (layers "B.Cu" "B.Paste" "B.Mask") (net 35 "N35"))
  (pad "D2" smd rect (at -2.29 -2.29) (size 1.06 1.06) (layers "B.Cu" "B.Paste" "B.Mask") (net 2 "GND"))
  (pad "D3" smd rect (at 0 -2.29) (size 1.06 1.06) (layers "B.Cu" "B.Paste" "B.Mask") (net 2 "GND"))
  (pad "D4" smd rect (at 2.29 -2.29) (size 1.06 1.06) (layers "B.Cu" "B.Paste" "B.Mask") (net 2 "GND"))
  (pad "D5" smd rect (at 4.58 -2.29) (size 1.06 1.06) (layers "B.Cu" "B.Paste" "B.Mask") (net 2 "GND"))
  (pad "E1" smd rect (at -4.58 -4.58) (size 1.06 1.06) (layers "B.Cu" "B.Paste" "B.Mask") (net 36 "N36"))
  (pad "E2" smd rect (at -2.29 -4.58) (size 1.06 1.06) (layers "B.Cu" "B.Paste" "B.Mask") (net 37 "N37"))
  (pad "E3" smd rect (at 0 -4.58) (size 1.06 1.06) (layers "B.Cu" "B.Paste" "B.Mask") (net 2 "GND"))
  (pad "E4" smd rect (at 2.29 -4.58) (size 1.06 1.06) (layers "B.Cu" "B.Paste" "B.Mask") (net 2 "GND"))
  (pad "E5" smd rect (at 4.58 -4.58) (size 1.06 1.06) (layers "B.Cu" "B.Paste" "B.Mask") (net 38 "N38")))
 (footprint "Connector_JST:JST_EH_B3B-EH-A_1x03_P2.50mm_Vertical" (layer "B.Cu") (at 61 48.674999 90)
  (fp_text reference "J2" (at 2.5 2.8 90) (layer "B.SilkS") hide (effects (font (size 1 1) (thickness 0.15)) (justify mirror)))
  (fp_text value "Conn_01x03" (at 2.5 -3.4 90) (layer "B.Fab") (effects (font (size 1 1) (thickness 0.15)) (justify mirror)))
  (pad "1" thru_hole roundrect (at 0 0 90) (size 1.7 1.95) (drill 0.95) (layers "*.Cu" "*.Mask") (roundrect_rratio 0.147059) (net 2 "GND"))
  (pad "2" thru_hole oval (at 2.5 0 90) (size 1.7 1.95) (drill 0.95) (layers "*.Cu" "*.Mask") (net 19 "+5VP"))
  (pad "3" thru_hole oval (at 5 0 90) (size 1.7 1.95) (drill 0.95) (layers "*.Cu" "*.Mask") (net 21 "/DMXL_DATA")))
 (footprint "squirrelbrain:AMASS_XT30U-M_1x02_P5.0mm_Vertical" (layer "B.Cu") (at 43.95 60.25)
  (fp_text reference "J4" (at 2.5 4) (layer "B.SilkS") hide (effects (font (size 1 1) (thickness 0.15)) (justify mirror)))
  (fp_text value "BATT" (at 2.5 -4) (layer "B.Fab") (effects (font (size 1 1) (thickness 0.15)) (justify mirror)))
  (pad "1" thru_hole rect (at 0 0) (size 3.8 3.8) (drill 2.7) (layers "*.Cu" "*.Mask") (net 2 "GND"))
  (pad "2" thru_hole circle (at 5 0) (size 3.8 3.8) (drill 2.7) (layers "*.Cu" "*.Mask") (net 27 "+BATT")))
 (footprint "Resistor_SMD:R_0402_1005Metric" (layer "B.Cu") (at 43.76 51.7 180)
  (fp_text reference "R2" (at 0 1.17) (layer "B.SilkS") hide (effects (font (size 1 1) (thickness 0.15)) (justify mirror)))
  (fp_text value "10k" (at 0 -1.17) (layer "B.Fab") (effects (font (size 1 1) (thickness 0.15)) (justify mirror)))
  (pad "1" smd roundrect (at -0.51 0 180) (size 0.54 0.64) (layers "B.Cu" "B.Paste" "B.Mask") (roundrect_rratio 0.25) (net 2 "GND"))
  (pad "2" smd roundrect (at 0.51 0 180) (size 0.54 0.64) (layers "B.Cu" "B.Paste" "B.Mask") (roundrect_rratio 0.25) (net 31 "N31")))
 (gr_line (start 63.5 61.313708) (end 63.5 38.686292) (stroke (width 0.15) (type solid)) (layer "Edge.Cuts"))
 (gr_circle (center 61.313708 38.686292) (end 62.413708 38.686292) (stroke (width 0.15) (type solid)) (fill none) (layer "Edge.Cuts"))
 (gr_arc (start 38.686292 63.5) (mid 37.140352 62.859648) (end 36.5 61.313708) (stroke (width 0.15) (type solid)) (layer "Edge.Cuts"))
 (gr_arc (start 36.5 38.686292) (mid 37.140352 37.140352) (end 38.686292 36.5) (stroke (width 0.15) (type solid)) (layer "Edge.Cuts"))
 (gr_line (start 61.313708 36.5) (end 38.686292 36.5) (stroke (width 0.15) (type solid)) (layer "Edge.Cuts"))
 (gr_arc (start 63.5 61.313708) (mid 62.859648 62.859648) (end 61.313708 63.5) (stroke (width 0.15) (type solid)) (layer "Edge.Cuts"))
 (gr_circle (center 38.686292 38.686292) (end 39.786292 38.686292) (stroke (width 0.15) (type solid)) (fill none) (layer "Edge.Cuts"))
 (gr_line (start 38.686292 63.5) (end 61.313708 63.5) (stroke (width 0.15) (type solid)) (layer "Edge.Cuts"))
 (gr_line (start 36.5 38.686292) (end 36.5 61.313708) (stroke (width 0.15) (type solid)) (layer "Edge.Cuts"))
 (gr_arc (start 61.313708 36.5) (mid 62.859648 37.140352) (end 63.5 38.686292) (stroke (width 0.15) (type solid)) (layer "Edge.Cuts"))
 (gr_circle (center 38.686292 61.313708) (end 39.786292 61.313708) (stroke (width 0.15) (type solid)) (fill none) (layer "Edge.Cuts"))
 (segment (start 61.160947 54.899105) (end 61.160947 54.253073) (width 0.2) (layer "F.Cu") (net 8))
 (segment (start 41.9375 52.08) (end 42.4175 51.6) (width 0.2) (layer "F.Cu") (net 8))
 (segment (start 60.060052 56) (end 61.160947 54.899105) (width 0.2) (layer "F.Cu") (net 8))
 (segment (start 57 56) (end 60.060052 56) (width 0.2) (layer "F.Cu") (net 8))
 (segment (start 52.6 51.6) (end 57 56) (width 0.2) (layer "F.Cu") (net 8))
 (segment (start 42.4175 51.6) (end 52.6 51.6) (width 0.2) (layer "F.Cu") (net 8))
 (via (at 61.160947 54.253073) (size 0.6) (drill 0.3) (layers "F.Cu" "B.Cu") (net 8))
 (segment (start 60.810052 53.300234) (end 60.334817 52.824999) (width 0.2) (layer "B.Cu") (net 8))
 (segment (start 60.810052 53.76) (end 60.810052 53.300234) (width 0.2) (layer "B.Cu") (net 8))
 (segment (start 60.334817 52.824999) (end 60.25 52.824999) (width 0.2) (layer "B.Cu") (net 8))
 (segment (start 61.160947 54.110895) (end 60.810052 53.76) (width 0.2) (layer "B.Cu") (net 8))
 (segment (start 61.310052 53.76) (end 60.810052 53.76) (width 0.2) (layer "B.Cu") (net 8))
 (segment (start 61.160947 54.253073) (end 61.160947 54.110895) (width 0.2) (layer "B.Cu") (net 8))
 (segment (start 56.5 56.5) (end 60.560052 56.5) (width 0.2) (layer "F.Cu") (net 9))
 (segment (start 41.9375 54.62) (end 44.5575 52) (width 0.2) (layer "F.Cu") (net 9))
 (segment (start 62.082098 54.977954) (end 62.082098 54.433127) (width 0.2) (layer "F.Cu") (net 9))
 (segment (start 60.560052 56.5) (end 62.082098 54.977954) (width 0.2) (layer "F.Cu") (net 9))
 (segment (start 44.5575 52) (end 52 52) (width 0.2) (layer "F.Cu") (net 9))
 (segment (start 52 52) (end 56.5 56.5) (width 0.2) (layer "F.Cu") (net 9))
 (via (at 62.082098 54.433127) (size 0.6) (drill 0.3) (layers "F.Cu" "B.Cu") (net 9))
 (segment (start 62.082098 54.433127) (end 62.082098 54.032046) (width 0.2) (layer "B.Cu") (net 9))
 (segment (start 62.082098 54.032046) (end 61.810052 53.76) (width 0.2) (layer "B.Cu") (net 9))
 (segment (start 58.1025 54.62) (end 58.868714 54.62) (width 0.2) (layer "F.Cu") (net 10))
 (segment (start 58.928766 54.62) (end 59.886163 53.662603) (width 0.2) (layer "F.Cu") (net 10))
 (via (at 59.886163 53.662603) (size 0.6) (drill 0.3) (layers "F.Cu" "B.Cu") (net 10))
 (segment (start 59.886163 53.662603) (end 60.212655 53.662603) (width 0.2) (layer "B.Cu") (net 10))
 (segment (start 60.212655 53.662603) (end 60.310052 53.76) (width 0.2) (layer "B.Cu") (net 10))
 (segment (start 60.486163 54.620043) (end 60.486163 53.633837) (width 0.2) (layer "F.Cu") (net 14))
 (segment (start 60.486163 53.633837) (end 60.67 53.45) (width 0.2) (layer "F.Cu") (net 14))
 (segment (start 60.006706 55.0995) (end 60.486163 54.620043) (width 0.2) (layer "F.Cu") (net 14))
 (via (at 60.006706 55.0995) (size 0.6) (drill 0.3) (layers "F.Cu" "B.Cu") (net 14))
 (segment (start 60.006706 55.0995) (end 60.147206 55.24) (width 0.2) (layer "B.Cu") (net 14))
 (segment (start 60.147206 55.24) (end 60.310052 55.24) (width 0.2) (layer "B.Cu") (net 14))
 (via (at 39.9 54.95) (size 0.6) (drill 0.3) (layers "F.Cu" "B.Cu") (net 2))
 (segment (start 39.7 55.154999) (end 39.7 55.15) (width 0.2) (layer "B.Cu") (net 2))
 (segment (start 39.7 55.15) (end 39.9 54.95) (width 0.2) (layer "B.Cu") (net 2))
 (via (at 51 55.5) (size 0.6) (drill 0.3) (layers "F.Cu" "B.Cu") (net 27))
 (via (at 49 53) (size 0.6) (drill 0.3) (layers "F.Cu" "B.Cu") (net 27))
 (via (at 50 53.5) (size 0.6) (drill 0.3) (layers "F.Cu" "B.Cu") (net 27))
 (via (at 49 55.5) (size 0.6) (drill 0.3) (layers "F.Cu" "B.Cu") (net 27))
 (via (at 51 53) (size 0.6) (drill 0.3) (layers "F.Cu" "B.Cu") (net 27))
 (via (at 50 55) (size 0.6) (drill 0.3) (layers "F.Cu" "B.Cu") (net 27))
 (segment (start 56.1 53.9) (end 56.1 53.225) (width 0.2) (layer "B.Cu") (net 22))
 (segment (start 61.185052 55.875) (end 59.775 55.875) (width 0.2) (layer "B.Cu") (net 22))
 (segment (start 56.5 54.3) (end 56.1 53.9) (width 0.2) (layer "B.Cu") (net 22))
 (segment (start 59.360052 55.460052) (end 59.360052 54.610052) (width 0.2) (layer "B.Cu") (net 22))
 (segment (start 59.05 54.3) (end 56.5 54.3) (width 0.2) (layer "B.Cu") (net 22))
 (segment (start 61.310052 55.24) (end 61.310052 55.75) (width 0.2) (layer "B.Cu") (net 22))
 (segment (start 59.360052 54.610052) (end 59.05 54.3) (width 0.2) (layer "B.Cu") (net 22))
 (segment (start 61.310052 55.75) (end 61.185052 55.875) (width 0.2) (layer "B.Cu") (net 22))
 (segment (start 59.775 55.875) (end 59.360052 55.460052) (width 0.2) (layer "B.Cu") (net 22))
 (segment (start 60.510052 54.45) (end 59.825737 54.45) (width 0.2) (layer "B.Cu") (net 23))
 (segment (start 60.810052 54.75) (end 60.510052 54.45) (width 0.2) (layer "B.Cu") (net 23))
 (segment (start 59.215685 53.9) (end 57.775 53.9) (width 0.2) (layer "B.Cu") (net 23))
 (segment (start 60.810052 55.24) (end 60.810052 54.75) (width 0.2) (layer "B.Cu") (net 23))
 (segment (start 57.775 53.9) (end 57.1 53.225) (width 0.2) (layer "B.Cu") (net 23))
 (segment (start 59.825737 54.45) (end 59.275737 53.9) (width 0.2) (layer "B.Cu") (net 23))
 (segment (start 39.665025 54.309999) (end 40.124315 54.309999) (width 0.2) (layer "B.Cu") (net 24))
 (segment (start 40.124315 54.309999) (end 41.209314 53.225) (width 0.2) (layer "B.Cu") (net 24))
 (segment (start 39.25 55.154999) (end 39.2 55.104999) (width 0.2) (layer "B.Cu") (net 24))
 (segment (start 39.2 54.775024) (end 39.665025 54.309999) (width 0.2) (layer "B.Cu") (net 24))
 (segment (start 39.2 55.104999) (end 39.2 54.775024) (width 0.2) (layer "B.Cu") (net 24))
 (segment (start 41.209314 53.225) (end 42.9 53.225) (width 0.2) (layer "B.Cu") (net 24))
 (segment (start 38.789999 55.789999) (end 40.5 55.789999) (width 0.2) (layer "B.Cu") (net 25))
 (segment (start 38.75 55.154999) (end 38.75 55.75) (width 0.2) (layer "B.Cu") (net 25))
 (segment (start 40.5 54.5) (end 40.7 54.3) (width 0.2) (layer "B.Cu") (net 25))
 (segment (start 40.7 54.3) (end 43.8 54.3) (width 0.2) (layer "B.Cu") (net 25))
 (segment (start 40.5 55.789999) (end 40.5 54.5) (width 0.2) (layer "B.Cu") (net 25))
 (segment (start 43.8 54.3) (end 43.9 54.2) (width 0.2) (layer "B.Cu") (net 25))
 (segment (start 43.9 54.2) (end 43.9 53.225) (width 0.2) (layer "B.Cu") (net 25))
 (segment (start 38.75 55.75) (end 38.789999 55.789999) (width 0.2) (layer "B.Cu") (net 25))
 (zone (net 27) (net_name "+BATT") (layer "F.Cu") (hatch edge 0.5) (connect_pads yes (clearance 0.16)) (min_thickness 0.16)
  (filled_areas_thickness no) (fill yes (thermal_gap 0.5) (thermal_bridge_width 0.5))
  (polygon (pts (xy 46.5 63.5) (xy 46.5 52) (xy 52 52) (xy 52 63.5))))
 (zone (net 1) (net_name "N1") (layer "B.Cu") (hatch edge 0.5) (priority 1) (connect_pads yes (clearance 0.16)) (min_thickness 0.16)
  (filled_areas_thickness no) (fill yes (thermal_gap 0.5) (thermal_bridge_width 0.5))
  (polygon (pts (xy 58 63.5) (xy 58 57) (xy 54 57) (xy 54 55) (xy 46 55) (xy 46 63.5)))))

